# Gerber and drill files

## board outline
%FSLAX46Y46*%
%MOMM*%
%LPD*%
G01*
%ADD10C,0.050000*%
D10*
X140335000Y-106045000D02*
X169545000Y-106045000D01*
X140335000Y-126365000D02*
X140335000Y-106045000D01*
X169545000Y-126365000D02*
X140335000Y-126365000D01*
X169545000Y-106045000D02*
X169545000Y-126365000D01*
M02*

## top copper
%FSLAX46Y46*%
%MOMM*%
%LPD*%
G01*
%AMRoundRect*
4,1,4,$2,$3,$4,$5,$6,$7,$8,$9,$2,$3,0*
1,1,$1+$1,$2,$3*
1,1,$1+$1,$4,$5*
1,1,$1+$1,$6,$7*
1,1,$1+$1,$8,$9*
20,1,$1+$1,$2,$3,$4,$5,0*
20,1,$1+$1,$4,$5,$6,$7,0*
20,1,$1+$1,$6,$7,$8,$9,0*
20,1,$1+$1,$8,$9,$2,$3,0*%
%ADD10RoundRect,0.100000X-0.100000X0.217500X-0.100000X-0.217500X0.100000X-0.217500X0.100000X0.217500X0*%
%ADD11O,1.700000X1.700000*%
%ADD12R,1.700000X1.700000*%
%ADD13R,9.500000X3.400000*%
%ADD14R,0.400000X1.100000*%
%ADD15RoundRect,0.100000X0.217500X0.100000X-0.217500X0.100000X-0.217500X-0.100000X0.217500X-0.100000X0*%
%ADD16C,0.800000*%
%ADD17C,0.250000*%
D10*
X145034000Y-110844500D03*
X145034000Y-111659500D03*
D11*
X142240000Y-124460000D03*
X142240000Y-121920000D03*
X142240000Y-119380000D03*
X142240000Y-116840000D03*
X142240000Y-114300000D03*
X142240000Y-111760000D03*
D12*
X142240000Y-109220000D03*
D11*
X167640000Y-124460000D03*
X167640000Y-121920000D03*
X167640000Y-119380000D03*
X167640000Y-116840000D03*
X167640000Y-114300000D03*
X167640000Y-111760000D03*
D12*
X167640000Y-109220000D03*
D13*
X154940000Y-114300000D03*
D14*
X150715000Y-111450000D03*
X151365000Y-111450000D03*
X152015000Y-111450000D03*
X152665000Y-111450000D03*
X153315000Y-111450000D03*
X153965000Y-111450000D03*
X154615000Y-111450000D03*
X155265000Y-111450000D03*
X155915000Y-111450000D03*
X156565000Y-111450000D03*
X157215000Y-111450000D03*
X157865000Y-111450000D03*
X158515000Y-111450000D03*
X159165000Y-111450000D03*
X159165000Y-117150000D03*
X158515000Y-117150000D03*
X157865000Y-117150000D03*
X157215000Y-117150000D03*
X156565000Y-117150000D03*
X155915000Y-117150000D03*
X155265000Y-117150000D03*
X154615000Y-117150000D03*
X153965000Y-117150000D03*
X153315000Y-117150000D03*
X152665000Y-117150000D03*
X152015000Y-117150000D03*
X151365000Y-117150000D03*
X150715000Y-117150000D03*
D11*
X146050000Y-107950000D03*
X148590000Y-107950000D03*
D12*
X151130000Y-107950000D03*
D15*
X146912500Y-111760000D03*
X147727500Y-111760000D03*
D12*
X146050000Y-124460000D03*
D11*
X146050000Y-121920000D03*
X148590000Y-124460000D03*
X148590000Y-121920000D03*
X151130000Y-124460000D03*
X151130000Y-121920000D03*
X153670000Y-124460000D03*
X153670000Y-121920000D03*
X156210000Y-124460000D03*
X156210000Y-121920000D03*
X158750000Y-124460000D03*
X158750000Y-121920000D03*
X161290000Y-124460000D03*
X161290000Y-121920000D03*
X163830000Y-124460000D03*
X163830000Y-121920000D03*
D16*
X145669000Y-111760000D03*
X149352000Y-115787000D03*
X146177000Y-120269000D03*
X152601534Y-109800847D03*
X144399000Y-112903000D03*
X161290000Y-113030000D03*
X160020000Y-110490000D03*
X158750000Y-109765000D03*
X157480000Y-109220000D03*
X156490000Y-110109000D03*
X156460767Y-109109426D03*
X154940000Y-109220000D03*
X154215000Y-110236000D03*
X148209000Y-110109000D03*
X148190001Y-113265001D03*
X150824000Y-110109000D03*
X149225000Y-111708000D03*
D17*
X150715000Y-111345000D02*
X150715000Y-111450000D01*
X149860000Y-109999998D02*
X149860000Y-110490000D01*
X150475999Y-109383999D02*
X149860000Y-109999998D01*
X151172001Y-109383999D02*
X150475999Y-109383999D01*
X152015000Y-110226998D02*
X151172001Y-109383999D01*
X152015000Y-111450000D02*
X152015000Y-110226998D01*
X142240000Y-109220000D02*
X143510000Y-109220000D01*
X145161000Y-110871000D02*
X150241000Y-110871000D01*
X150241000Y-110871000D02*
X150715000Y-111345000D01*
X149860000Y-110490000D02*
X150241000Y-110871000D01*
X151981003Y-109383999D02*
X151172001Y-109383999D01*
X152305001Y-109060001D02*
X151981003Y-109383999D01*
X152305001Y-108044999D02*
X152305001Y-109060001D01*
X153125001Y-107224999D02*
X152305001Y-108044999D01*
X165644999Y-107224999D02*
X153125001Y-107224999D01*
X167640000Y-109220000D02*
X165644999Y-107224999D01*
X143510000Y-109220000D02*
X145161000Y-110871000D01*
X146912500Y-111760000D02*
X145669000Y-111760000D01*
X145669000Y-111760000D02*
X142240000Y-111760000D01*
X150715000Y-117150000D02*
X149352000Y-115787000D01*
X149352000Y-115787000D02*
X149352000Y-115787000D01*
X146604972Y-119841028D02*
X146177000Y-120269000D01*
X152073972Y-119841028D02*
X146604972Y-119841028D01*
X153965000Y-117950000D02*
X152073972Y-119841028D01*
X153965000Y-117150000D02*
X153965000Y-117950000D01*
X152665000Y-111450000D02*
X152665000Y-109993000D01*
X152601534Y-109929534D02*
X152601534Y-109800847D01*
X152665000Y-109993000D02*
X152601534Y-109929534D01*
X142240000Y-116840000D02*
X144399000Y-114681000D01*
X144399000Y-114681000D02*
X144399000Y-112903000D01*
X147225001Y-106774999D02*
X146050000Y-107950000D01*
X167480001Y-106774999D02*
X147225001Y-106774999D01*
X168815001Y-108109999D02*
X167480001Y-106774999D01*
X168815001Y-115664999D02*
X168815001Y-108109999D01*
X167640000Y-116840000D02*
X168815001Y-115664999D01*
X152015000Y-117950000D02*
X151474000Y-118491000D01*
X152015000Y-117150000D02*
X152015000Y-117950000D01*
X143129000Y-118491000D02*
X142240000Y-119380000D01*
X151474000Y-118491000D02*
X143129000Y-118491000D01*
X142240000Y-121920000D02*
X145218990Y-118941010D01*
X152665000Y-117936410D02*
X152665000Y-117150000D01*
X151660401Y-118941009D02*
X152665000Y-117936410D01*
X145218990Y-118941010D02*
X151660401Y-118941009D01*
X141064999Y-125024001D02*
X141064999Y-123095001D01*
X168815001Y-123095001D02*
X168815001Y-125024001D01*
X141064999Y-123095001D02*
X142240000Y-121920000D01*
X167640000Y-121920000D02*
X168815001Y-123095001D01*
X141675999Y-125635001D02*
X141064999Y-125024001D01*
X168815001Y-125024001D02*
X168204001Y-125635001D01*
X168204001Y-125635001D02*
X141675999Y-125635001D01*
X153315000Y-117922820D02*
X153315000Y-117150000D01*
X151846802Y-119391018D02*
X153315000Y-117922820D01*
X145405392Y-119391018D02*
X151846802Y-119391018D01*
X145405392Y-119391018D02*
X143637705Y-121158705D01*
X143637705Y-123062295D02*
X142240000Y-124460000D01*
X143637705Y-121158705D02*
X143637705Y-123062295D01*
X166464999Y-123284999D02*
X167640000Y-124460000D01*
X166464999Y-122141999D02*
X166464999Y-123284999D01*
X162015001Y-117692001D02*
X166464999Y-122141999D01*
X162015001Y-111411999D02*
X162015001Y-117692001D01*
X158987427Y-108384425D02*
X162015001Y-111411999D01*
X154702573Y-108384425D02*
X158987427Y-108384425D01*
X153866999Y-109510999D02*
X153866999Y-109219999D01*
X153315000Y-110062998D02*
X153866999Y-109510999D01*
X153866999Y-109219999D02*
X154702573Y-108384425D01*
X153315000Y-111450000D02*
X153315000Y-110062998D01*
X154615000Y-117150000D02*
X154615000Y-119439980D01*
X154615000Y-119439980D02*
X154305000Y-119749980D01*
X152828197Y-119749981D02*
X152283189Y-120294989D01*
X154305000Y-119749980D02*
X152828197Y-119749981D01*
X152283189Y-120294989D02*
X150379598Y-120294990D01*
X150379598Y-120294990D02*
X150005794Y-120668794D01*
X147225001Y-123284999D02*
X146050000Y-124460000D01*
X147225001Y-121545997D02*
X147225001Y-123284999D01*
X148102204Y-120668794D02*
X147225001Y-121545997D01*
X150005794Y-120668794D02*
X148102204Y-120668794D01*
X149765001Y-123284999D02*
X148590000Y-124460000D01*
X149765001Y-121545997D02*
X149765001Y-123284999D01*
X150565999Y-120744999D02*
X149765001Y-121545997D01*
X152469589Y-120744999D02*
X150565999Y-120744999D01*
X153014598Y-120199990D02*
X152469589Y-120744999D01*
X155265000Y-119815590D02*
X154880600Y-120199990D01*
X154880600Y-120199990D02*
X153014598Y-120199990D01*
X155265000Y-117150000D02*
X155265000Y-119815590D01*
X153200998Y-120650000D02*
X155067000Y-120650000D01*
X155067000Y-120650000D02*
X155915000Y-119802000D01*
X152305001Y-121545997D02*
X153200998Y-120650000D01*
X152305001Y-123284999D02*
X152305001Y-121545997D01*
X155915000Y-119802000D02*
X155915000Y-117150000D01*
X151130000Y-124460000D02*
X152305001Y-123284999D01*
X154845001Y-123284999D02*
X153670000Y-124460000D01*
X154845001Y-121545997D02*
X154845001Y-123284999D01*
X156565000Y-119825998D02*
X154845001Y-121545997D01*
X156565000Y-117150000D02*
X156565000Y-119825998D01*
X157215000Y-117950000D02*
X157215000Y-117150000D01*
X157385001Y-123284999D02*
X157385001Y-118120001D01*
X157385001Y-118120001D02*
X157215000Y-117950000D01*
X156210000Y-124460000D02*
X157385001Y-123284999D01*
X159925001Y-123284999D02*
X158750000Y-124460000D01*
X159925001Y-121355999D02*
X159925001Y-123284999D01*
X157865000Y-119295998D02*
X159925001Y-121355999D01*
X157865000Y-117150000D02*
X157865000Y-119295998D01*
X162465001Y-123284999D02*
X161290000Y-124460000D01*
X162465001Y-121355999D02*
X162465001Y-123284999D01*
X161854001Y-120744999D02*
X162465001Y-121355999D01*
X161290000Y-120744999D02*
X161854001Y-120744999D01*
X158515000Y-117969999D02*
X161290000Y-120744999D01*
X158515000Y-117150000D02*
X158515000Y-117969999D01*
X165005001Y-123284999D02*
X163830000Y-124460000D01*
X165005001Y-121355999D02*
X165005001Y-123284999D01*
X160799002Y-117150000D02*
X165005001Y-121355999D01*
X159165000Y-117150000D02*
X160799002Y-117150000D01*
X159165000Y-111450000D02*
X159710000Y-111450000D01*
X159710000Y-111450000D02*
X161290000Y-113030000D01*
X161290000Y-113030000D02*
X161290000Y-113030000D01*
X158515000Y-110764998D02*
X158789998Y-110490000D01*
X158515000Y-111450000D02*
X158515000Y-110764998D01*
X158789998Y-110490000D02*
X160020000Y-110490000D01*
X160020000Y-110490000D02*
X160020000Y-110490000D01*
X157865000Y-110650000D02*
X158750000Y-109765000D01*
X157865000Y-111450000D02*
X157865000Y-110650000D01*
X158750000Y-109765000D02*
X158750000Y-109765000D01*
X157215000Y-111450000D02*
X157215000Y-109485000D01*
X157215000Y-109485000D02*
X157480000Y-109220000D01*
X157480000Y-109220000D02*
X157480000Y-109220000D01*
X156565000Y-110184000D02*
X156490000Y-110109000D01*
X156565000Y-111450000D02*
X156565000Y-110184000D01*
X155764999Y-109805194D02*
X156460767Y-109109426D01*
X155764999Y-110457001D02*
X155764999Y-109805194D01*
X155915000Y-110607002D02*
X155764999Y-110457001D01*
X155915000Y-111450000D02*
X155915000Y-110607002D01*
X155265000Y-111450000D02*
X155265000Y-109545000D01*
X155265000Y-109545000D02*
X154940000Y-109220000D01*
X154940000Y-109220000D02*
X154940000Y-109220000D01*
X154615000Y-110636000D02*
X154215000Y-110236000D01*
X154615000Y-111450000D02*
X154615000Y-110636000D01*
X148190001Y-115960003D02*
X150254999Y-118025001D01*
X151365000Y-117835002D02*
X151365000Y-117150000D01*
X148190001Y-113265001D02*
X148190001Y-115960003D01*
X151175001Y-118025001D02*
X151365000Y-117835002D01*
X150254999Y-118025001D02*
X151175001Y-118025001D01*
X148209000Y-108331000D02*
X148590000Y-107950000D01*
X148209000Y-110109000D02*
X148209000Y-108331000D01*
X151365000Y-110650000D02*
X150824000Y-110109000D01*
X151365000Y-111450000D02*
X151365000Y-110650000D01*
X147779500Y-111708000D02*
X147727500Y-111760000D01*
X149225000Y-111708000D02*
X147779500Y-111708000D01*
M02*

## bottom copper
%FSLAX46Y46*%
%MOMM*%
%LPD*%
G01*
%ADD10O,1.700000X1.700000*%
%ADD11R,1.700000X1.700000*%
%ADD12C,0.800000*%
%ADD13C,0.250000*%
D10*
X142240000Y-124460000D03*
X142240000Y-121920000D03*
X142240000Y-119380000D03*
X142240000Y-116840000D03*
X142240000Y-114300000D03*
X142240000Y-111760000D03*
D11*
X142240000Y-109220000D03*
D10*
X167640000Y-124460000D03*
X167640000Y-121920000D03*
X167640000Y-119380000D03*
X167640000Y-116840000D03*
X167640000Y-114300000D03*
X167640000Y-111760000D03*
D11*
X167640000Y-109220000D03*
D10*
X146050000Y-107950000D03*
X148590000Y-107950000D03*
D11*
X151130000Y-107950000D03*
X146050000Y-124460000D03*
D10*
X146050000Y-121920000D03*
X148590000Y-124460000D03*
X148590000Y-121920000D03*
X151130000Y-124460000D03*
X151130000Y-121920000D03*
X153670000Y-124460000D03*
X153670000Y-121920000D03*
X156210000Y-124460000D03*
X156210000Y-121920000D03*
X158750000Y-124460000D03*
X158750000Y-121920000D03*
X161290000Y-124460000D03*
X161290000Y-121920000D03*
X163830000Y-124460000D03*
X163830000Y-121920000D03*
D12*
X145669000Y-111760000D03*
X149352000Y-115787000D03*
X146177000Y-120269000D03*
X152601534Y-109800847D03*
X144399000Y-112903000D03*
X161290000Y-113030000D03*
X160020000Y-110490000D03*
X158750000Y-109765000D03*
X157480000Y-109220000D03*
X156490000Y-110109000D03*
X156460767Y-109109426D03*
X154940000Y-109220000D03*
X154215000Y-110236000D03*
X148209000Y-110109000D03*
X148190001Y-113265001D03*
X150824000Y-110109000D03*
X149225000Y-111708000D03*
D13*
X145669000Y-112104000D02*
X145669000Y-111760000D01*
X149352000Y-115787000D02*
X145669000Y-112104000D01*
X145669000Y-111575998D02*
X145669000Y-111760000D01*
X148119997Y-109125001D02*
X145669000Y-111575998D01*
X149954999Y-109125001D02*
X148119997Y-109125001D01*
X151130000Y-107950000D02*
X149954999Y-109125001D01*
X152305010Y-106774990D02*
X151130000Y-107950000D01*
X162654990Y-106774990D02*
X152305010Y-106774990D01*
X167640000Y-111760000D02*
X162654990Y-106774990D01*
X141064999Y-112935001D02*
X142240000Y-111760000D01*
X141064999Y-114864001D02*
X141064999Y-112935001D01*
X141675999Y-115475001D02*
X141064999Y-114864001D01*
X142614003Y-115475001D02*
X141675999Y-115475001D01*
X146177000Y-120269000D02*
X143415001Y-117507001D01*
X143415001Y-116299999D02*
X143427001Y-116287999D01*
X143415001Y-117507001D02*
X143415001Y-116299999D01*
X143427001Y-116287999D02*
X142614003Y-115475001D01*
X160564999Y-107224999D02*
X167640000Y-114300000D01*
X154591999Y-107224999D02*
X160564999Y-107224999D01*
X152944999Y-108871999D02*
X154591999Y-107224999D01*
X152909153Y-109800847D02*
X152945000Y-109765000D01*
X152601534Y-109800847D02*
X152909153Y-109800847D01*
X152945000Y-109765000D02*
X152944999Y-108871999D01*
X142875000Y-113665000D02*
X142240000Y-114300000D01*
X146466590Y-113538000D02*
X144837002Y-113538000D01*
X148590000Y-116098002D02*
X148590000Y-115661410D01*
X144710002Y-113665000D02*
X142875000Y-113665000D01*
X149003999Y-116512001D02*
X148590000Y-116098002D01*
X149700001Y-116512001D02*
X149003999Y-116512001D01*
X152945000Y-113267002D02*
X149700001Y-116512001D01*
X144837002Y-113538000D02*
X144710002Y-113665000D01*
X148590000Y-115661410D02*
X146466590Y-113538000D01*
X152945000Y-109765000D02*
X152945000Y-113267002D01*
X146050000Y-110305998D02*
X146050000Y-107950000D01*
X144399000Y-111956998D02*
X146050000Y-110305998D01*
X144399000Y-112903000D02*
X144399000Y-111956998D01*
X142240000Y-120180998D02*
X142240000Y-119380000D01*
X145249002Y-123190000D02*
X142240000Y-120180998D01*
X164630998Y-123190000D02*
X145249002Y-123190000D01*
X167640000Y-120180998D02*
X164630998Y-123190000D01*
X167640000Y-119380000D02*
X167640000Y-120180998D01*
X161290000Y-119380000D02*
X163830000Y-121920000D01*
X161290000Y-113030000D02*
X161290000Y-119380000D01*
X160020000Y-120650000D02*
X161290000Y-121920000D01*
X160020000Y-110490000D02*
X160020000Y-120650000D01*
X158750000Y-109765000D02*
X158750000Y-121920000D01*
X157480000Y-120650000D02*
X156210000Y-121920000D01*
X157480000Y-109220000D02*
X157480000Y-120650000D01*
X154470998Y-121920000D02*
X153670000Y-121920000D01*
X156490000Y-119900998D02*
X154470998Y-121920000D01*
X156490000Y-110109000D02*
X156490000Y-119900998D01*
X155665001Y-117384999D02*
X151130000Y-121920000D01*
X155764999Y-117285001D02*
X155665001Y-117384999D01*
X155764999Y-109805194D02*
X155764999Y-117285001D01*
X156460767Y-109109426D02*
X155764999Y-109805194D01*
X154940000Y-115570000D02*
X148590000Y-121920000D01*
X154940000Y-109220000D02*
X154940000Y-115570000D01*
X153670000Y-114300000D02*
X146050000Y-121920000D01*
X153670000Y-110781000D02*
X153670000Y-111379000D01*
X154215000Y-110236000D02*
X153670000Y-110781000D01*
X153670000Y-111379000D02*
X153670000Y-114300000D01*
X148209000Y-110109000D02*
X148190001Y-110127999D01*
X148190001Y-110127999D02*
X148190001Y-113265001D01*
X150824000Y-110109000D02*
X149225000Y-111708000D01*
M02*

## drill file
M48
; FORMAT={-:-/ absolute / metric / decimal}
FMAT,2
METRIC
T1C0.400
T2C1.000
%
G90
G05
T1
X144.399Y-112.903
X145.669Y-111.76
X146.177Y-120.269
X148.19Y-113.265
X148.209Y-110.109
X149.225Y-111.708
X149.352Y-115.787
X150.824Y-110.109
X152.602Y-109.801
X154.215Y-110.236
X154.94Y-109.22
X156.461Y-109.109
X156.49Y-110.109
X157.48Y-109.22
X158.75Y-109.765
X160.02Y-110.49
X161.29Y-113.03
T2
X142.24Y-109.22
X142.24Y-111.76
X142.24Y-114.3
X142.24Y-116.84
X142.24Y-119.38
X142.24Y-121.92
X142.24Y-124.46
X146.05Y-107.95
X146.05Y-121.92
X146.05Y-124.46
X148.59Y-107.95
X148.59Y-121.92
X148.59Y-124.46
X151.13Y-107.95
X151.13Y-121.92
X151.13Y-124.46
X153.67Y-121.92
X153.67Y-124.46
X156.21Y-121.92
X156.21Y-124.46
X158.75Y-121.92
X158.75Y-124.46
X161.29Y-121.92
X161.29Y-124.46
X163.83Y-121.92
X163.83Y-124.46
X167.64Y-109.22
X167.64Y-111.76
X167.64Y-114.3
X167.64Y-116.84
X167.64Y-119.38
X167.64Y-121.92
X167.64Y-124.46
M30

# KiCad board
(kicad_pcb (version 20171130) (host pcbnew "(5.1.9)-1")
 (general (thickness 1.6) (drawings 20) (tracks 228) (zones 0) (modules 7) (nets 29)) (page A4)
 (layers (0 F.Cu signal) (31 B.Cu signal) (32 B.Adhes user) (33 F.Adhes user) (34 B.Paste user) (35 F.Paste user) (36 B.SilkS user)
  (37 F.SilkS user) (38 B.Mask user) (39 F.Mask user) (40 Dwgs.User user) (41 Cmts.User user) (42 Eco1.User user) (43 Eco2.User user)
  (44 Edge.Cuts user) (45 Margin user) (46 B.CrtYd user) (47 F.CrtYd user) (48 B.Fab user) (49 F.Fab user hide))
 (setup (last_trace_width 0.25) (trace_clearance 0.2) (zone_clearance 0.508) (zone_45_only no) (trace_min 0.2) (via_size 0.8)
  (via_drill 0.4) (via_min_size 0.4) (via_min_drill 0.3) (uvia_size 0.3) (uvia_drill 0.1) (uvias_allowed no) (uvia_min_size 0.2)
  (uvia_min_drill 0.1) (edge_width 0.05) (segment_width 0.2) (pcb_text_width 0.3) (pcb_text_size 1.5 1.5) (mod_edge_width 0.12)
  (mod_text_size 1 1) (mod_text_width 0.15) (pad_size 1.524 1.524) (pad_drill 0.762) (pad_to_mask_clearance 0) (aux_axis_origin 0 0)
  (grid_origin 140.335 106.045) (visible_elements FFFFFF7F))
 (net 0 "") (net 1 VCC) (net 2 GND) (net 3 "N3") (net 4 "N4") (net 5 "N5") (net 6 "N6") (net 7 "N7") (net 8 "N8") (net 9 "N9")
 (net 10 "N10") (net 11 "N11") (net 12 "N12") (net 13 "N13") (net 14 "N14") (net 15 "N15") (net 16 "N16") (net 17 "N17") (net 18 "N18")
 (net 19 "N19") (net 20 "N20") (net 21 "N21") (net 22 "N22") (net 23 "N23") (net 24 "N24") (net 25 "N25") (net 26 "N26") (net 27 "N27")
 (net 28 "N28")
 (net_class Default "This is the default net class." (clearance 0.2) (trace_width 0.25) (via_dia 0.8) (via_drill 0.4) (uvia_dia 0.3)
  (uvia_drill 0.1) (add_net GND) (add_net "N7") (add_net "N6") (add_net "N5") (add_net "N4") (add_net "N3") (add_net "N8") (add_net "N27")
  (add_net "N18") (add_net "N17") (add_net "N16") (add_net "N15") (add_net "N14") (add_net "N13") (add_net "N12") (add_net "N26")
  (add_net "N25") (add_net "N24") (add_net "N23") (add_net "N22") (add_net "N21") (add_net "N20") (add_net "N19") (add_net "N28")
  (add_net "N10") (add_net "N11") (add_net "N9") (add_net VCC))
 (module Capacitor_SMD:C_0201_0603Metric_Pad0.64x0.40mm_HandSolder (layer F.Cu) (at 145.034 111.252 270)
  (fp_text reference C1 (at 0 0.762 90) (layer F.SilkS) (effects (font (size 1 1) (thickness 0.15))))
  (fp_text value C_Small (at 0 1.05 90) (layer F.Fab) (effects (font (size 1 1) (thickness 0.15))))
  (pad "" smd roundrect (at -0.4325 0 270) (size 0.458 0.36) (layers F.Paste) (roundrect_rratio 0.25))
  (pad "" smd roundrect (at 0.4325 0 270) (size 0.458 0.36) (layers F.Paste) (roundrect_rratio 0.25))
  (pad 1 smd roundrect (at -0.4075 0 270) (size 0.635 0.4) (layers F.Cu F.Mask) (roundrect_rratio 0.25) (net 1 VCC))
  (pad 2 smd roundrect (at 0.4075 0 270) (size 0.635 0.4) (layers F.Cu F.Mask) (roundrect_rratio 0.25) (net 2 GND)))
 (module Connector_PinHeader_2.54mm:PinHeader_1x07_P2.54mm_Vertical (layer F.Cu) (at 142.24 109.22)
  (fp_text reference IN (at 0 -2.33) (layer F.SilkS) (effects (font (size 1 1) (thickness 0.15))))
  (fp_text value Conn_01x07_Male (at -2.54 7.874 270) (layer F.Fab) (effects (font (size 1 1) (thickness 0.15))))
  (pad 7 thru_hole oval (at 0 15.24) (size 1.7 1.7) (drill 1) (layers *.Cu *.Mask) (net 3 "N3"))
  (pad 6 thru_hole oval (at 0 12.7) (size 1.7 1.7) (drill 1) (layers *.Cu *.Mask) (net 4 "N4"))
  (pad 5 thru_hole oval (at 0 10.16) (size 1.7 1.7) (drill 1) (layers *.Cu *.Mask) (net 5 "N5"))
  (pad 4 thru_hole oval (at 0 7.62) (size 1.7 1.7) (drill 1) (layers *.Cu *.Mask) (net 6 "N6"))
  (pad 3 thru_hole oval (at 0 5.08) (size 1.7 1.7) (drill 1) (layers *.Cu *.Mask) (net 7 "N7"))
  (pad 2 thru_hole oval (at 0 2.54) (size 1.7 1.7) (drill 1) (layers *.Cu *.Mask) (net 2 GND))
  (pad 1 thru_hole rect (at 0 0) (size 1.7 1.7) (drill 1) (layers *.Cu *.Mask) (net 1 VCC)))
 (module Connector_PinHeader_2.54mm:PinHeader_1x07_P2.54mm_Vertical (layer F.Cu) (at 167.64 109.22)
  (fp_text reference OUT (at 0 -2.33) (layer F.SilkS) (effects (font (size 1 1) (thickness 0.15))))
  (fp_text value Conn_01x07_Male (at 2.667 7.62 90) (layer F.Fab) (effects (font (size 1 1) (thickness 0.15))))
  (pad 7 thru_hole oval (at 0 15.24) (size 1.7 1.7) (drill 1) (layers *.Cu *.Mask) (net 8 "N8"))
  (pad 6 thru_hole oval (at 0 12.7) (size 1.7 1.7) (drill 1) (layers *.Cu *.Mask) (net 4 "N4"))
  (pad 5 thru_hole oval (at 0 10.16) (size 1.7 1.7) (drill 1) (layers *.Cu *.Mask) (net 5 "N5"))
  (pad 4 thru_hole oval (at 0 7.62) (size 1.7 1.7) (drill 1) (layers *.Cu *.Mask) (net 6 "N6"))
  (pad 3 thru_hole oval (at 0 5.08) (size 1.7 1.7) (drill 1) (layers *.Cu *.Mask) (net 7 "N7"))
  (pad 2 thru_hole oval (at 0 2.54) (size 1.7 1.7) (drill 1) (layers *.Cu *.Mask) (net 2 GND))
  (pad 1 thru_hole rect (at 0 0) (size 1.7 1.7) (drill 1) (layers *.Cu *.Mask) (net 1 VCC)))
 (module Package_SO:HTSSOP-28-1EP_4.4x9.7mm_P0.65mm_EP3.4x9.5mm (layer F.Cu) (at 154.94 114.3 90)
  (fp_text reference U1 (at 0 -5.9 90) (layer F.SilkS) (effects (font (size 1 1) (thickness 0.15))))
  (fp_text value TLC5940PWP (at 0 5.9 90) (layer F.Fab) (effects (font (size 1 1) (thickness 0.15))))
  (pad "" smd rect (at -0.85 3.8 90) (size 1.4 1.6) (layers F.Paste))
  (pad "" smd rect (at 0.85 3.8 90) (size 1.4 1.6) (layers F.Paste))
  (pad "" smd rect (at -0.85 1.9 90) (size 1.4 1.6) (layers F.Paste))
  (pad "" smd rect (at 0.85 1.9 90) (size 1.4 1.6) (layers F.Paste))
  (pad "" smd rect (at -0.85 0 90) (size 1.4 1.6) (layers F.Paste))
  (pad "" smd rect (at 0.85 0 90) (size 1.4 1.6) (layers F.Paste))
  (pad "" smd rect (at -0.85 -1.9 90) (size 1.4 1.6) (layers F.Paste))
  (pad "" smd rect (at 0.85 -1.9 90) (size 1.4 1.6) (layers F.Paste))
  (pad "" smd rect (at 0.85 -3.8 90) (size 1.4 1.6) (layers F.Paste))
  (pad "" smd rect (at -0.85 -3.8 90) (size 1.4 1.6) (layers F.Paste))
  (pad 29 smd rect (at 0 0 90) (size 3.4 9.5) (layers F.Cu F.Mask) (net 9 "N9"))
  (pad 28 smd rect (at 2.85 -4.225 90) (size 1.1 0.4) (layers F.Cu F.Paste F.Mask) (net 1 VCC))
  (pad 27 smd rect (at 2.85 -3.575 90) (size 1.1 0.4) (layers F.Cu F.Paste F.Mask) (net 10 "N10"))
  (pad 26 smd rect (at 2.85 -2.925 90) (size 1.1 0.4) (layers F.Cu F.Paste F.Mask) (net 1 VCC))
  (pad 25 smd rect (at 2.85 -2.275 90) (size 1.1 0.4) (layers F.Cu F.Paste F.Mask) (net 7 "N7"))
  (pad 24 smd rect (at 2.85 -1.625 90) (size 1.1 0.4) (layers F.Cu F.Paste F.Mask) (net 8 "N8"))
  (pad 23 smd rect (at 2.85 -0.975 90) (size 1.1 0.4) (layers F.Cu F.Paste F.Mask) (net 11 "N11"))
  (pad 22 smd rect (at 2.85 -0.325 90) (size 1.1 0.4) (layers F.Cu F.Paste F.Mask) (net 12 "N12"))
  (pad 21 smd rect (at 2.85 0.325 90) (size 1.1 0.4) (layers F.Cu F.Paste F.Mask) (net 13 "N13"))
  (pad 20 smd rect (at 2.85 0.975 90) (size 1.1 0.4) (layers F.Cu F.Paste F.Mask) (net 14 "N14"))
  (pad 19 smd rect (at 2.85 1.625 90) (size 1.1 0.4) (layers F.Cu F.Paste F.Mask) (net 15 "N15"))
  (pad 18 smd rect (at 2.85 2.275 90) (size 1.1 0.4) (layers F.Cu F.Paste F.Mask) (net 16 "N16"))
  (pad 17 smd rect (at 2.85 2.925 90) (size 1.1 0.4) (layers F.Cu F.Paste F.Mask) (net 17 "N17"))
  (pad 16 smd rect (at 2.85 3.575 90) (size 1.1 0.4) (layers F.Cu F.Paste F.Mask) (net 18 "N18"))
  (pad 15 smd rect (at 2.85 4.225 90) (size 1.1 0.4) (layers F.Cu F.Paste F.Mask) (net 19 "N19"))
  (pad 14 smd rect (at -2.85 4.225 90) (size 1.1 0.4) (layers F.Cu F.Paste F.Mask) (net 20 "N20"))
  (pad 13 smd rect (at -2.85 3.575 90) (size 1.1 0.4) (layers F.Cu F.Paste F.Mask) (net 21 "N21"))
  (pad 12 smd rect (at -2.85 2.925 90) (size 1.1 0.4) (layers F.Cu F.Paste F.Mask) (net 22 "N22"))
  (pad 11 smd rect (at -2.85 2.275 90) (size 1.1 0.4) (layers F.Cu F.Paste F.Mask) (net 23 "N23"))
  (pad 10 smd rect (at -2.85 1.625 90) (size 1.1 0.4) (layers F.Cu F.Paste F.Mask) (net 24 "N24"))
  (pad 9 smd rect (at -2.85 0.975 90) (size 1.1 0.4) (layers F.Cu F.Paste F.Mask) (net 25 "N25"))
  (pad 8 smd rect (at -2.85 0.325 90) (size 1.1 0.4) (layers F.Cu F.Paste F.Mask) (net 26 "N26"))
  (pad 7 smd rect (at -2.85 -0.325 90) (size 1.1 0.4) (layers F.Cu F.Paste F.Mask) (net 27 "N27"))
  (pad 6 smd rect (at -2.85 -0.975 90) (size 1.1 0.4) (layers F.Cu F.Paste F.Mask) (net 2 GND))
  (pad 5 smd rect (at -2.85 -1.625 90) (size 1.1 0.4) (layers F.Cu F.Paste F.Mask) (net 3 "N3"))
  (pad 4 smd rect (at -2.85 -2.275 90) (size 1.1 0.4) (layers F.Cu F.Paste F.Mask) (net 4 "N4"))
  (pad 3 smd rect (at -2.85 -2.925 90) (size 1.1 0.4) (layers F.Cu F.Paste F.Mask) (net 5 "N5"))
  (pad 2 smd rect (at -2.85 -3.575 90) (size 1.1 0.4) (layers F.Cu F.Paste F.Mask) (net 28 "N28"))
  (pad 1 smd rect (at -2.85 -4.225 90) (size 1.1 0.4) (layers F.Cu F.Paste F.Mask) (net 2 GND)))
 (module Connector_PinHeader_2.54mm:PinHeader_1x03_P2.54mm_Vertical (layer F.Cu) (at 151.13 107.95 270)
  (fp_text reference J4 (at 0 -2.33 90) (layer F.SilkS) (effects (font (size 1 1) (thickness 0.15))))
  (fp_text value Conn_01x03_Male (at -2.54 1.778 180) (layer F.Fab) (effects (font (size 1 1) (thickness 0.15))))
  (pad 3 thru_hole oval (at 0 5.08 270) (size 1.7 1.7) (drill 1) (layers *.Cu *.Mask) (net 6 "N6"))
  (pad 2 thru_hole oval (at 0 2.54 270) (size 1.7 1.7) (drill 1) (layers *.Cu *.Mask) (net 28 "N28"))
  (pad 1 thru_hole rect (at 0 0 270) (size 1.7 1.7) (drill 1) (layers *.Cu *.Mask) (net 2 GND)))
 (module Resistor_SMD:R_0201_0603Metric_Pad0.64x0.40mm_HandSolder (layer F.Cu) (at 147.32 111.76 180)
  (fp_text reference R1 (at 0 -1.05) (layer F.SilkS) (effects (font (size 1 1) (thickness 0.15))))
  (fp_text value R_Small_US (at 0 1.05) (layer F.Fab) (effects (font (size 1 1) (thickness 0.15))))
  (pad 2 smd roundrect (at 0.4075 0 180) (size 0.635 0.4) (layers F.Cu F.Mask) (roundrect_rratio 0.25) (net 2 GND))
  (pad 1 smd roundrect (at -0.4075 0 180) (size 0.635 0.4) (layers F.Cu F.Mask) (roundrect_rratio 0.25) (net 10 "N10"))
  (pad "" smd roundrect (at 0.4325 0 180) (size 0.458 0.36) (layers F.Paste) (roundrect_rratio 0.25))
  (pad "" smd roundrect (at -0.4325 0 180) (size 0.458 0.36) (layers F.Paste) (roundrect_rratio 0.25)))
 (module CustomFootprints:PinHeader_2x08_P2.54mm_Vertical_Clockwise (layer F.Cu) (at 146.05 124.46 90)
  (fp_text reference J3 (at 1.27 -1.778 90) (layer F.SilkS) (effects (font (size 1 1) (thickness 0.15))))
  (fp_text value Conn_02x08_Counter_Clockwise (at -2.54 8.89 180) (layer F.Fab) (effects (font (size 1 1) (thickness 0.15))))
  (pad 1 thru_hole rect (at 0 0 90) (size 1.7 1.7) (drill 1) (layers *.Cu *.Mask) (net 27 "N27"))
  (pad 16 thru_hole oval (at 2.54 0 90) (size 1.7 1.7) (drill 1) (layers *.Cu *.Mask) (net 12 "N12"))
  (pad 2 thru_hole oval (at 0 2.54 90) (size 1.7 1.7) (drill 1) (layers *.Cu *.Mask) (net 26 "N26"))
  (pad 15 thru_hole oval (at 2.54 2.54 90) (size 1.7 1.7) (drill 1) (layers *.Cu *.Mask) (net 13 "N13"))
  (pad 3 thru_hole oval (at 0 5.08 90) (size 1.7 1.7) (drill 1) (layers *.Cu *.Mask) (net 25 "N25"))
  (pad 14 thru_hole oval (at 2.54 5.08 90) (size 1.7 1.7) (drill 1) (layers *.Cu *.Mask) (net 14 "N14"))
  (pad 4 thru_hole oval (at 0 7.62 90) (size 1.7 1.7) (drill 1) (layers *.Cu *.Mask) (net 24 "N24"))
  (pad 13 thru_hole oval (at 2.54 7.62 90) (size 1.7 1.7) (drill 1) (layers *.Cu *.Mask) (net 15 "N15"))
  (pad 5 thru_hole oval (at 0 10.16 90) (size 1.7 1.7) (drill 1) (layers *.Cu *.Mask) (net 23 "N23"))
  (pad 12 thru_hole oval (at 2.54 10.16 90) (size 1.7 1.7) (drill 1) (layers *.Cu *.Mask) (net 16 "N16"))
  (pad 6 thru_hole oval (at 0 12.7 90) (size 1.7 1.7) (drill 1) (layers *.Cu *.Mask) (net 22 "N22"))
  (pad 11 thru_hole oval (at 2.54 12.7 90) (size 1.7 1.7) (drill 1) (layers *.Cu *.Mask) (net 17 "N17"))
  (pad 7 thru_hole oval (at 0 15.24 90) (size 1.7 1.7) (drill 1) (layers *.Cu *.Mask) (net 21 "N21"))
  (pad 10 thru_hole oval (at 2.54 15.24 90) (size 1.7 1.7) (drill 1) (layers *.Cu *.Mask) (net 18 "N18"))
  (pad 8 thru_hole oval (at 0 17.78 90) (size 1.7 1.7) (drill 1) (layers *.Cu *.Mask) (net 20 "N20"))
  (pad 9 thru_hole oval (at 2.54 17.78 90) (size 1.7 1.7) (drill 1) (layers *.Cu *.Mask) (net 19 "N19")))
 (gr_line (start 140.335 106.045) (end 169.545 106.045) (layer Edge.Cuts) (width 0.05))
 (gr_line (start 140.335 126.365) (end 140.335 106.045) (layer Edge.Cuts) (width 0.05))
 (gr_line (start 169.545 126.365) (end 140.335 126.365) (layer Edge.Cuts) (width 0.05))
 (gr_line (start 169.545 106.045) (end 169.545 126.365) (layer Edge.Cuts) (width 0.05))
 (segment (start 150.715 111.345) (end 150.715 111.45) (width 0.25) (layer F.Cu) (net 1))
 (segment (start 149.86 109.999998) (end 149.86 110.49) (width 0.25) (layer F.Cu) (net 1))
 (segment (start 150.475999 109.383999) (end 149.86 109.999998) (width 0.25) (layer F.Cu) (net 1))
 (segment (start 151.172001 109.383999) (end 150.475999 109.383999) (width 0.25) (layer F.Cu) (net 1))
 (segment (start 152.015 110.226998) (end 151.172001 109.383999) (width 0.25) (layer F.Cu) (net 1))
 (segment (start 152.015 111.45) (end 152.015 110.226998) (width 0.25) (layer F.Cu) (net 1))
 (segment (start 142.24 109.22) (end 143.51 109.22) (width 0.25) (layer F.Cu) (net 1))
 (segment (start 145.161 110.871) (end 150.241 110.871) (width 0.25) (layer F.Cu) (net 1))
 (segment (start 150.241 110.871) (end 150.715 111.345) (width 0.25) (layer F.Cu) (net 1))
 (segment (start 149.86 110.49) (end 150.241 110.871) (width 0.25) (layer F.Cu) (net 1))
 (segment (start 151.981003 109.383999) (end 151.172001 109.383999) (width 0.25) (layer F.Cu) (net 1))
 (segment (start 152.305001 109.060001) (end 151.981003 109.383999) (width 0.25) (layer F.Cu) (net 1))
 (segment (start 152.305001 108.044999) (end 152.305001 109.060001) (width 0.25) (layer F.Cu) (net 1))
 (segment (start 153.125001 107.224999) (end 152.305001 108.044999) (width 0.25) (layer F.Cu) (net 1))
 (segment (start 165.644999 107.224999) (end 153.125001 107.224999) (width 0.25) (layer F.Cu) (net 1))
 (segment (start 167.64 109.22) (end 165.644999 107.224999) (width 0.25) (layer F.Cu) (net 1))
 (segment (start 143.51 109.22) (end 145.161 110.871) (width 0.25) (layer F.Cu) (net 1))
 (segment (start 146.9125 111.76) (end 145.669 111.76) (width 0.25) (layer F.Cu) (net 2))
 (segment (start 145.669 111.76) (end 142.24 111.76) (width 0.25) (layer F.Cu) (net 2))
 (via (at 145.669 111.76) (size 0.8) (drill 0.4) (layers F.Cu B.Cu) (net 2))
 (segment (start 150.715 117.15) (end 149.352 115.787) (width 0.25) (layer F.Cu) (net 2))
 (segment (start 149.352 115.787) (end 149.352 115.787) (width 0.25) (layer F.Cu) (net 2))
 (via (at 149.352 115.787) (size 0.8) (drill 0.4) (layers F.Cu B.Cu) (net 2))
 (segment (start 145.669 112.104) (end 145.669 111.76) (width 0.25) (layer B.Cu) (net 2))
 (segment (start 149.352 115.787) (end 145.669 112.104) (width 0.25) (layer B.Cu) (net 2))
 (segment (start 145.669 111.575998) (end 145.669 111.76) (width 0.25) (layer B.Cu) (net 2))
 (segment (start 148.119997 109.125001) (end 145.669 111.575998) (width 0.25) (layer B.Cu) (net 2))
 (segment (start 149.954999 109.125001) (end 148.119997 109.125001) (width 0.25) (layer B.Cu) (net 2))
 (segment (start 151.13 107.95) (end 149.954999 109.125001) (width 0.25) (layer B.Cu) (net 2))
 (segment (start 152.30501 106.77499) (end 151.13 107.95) (width 0.25) (layer B.Cu) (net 2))
 (segment (start 162.65499 106.77499) (end 152.30501 106.77499) (width 0.25) (layer B.Cu) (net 2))
 (segment (start 167.64 111.76) (end 162.65499 106.77499) (width 0.25) (layer B.Cu) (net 2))
 (segment (start 146.604972 119.841028) (end 146.177 120.269) (width 0.25) (layer F.Cu) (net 2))
 (segment (start 152.073972 119.841028) (end 146.604972 119.841028) (width 0.25) (layer F.Cu) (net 2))
 (segment (start 153.965 117.95) (end 152.073972 119.841028) (width 0.25) (layer F.Cu) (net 2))
 (via (at 146.177 120.269) (size 0.8) (drill 0.4) (layers F.Cu B.Cu) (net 2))
 (segment (start 153.965 117.15) (end 153.965 117.95) (width 0.25) (layer F.Cu) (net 2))
 (segment (start 141.064999 112.935001) (end 142.24 111.76) (width 0.25) (layer B.Cu) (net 2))
 (segment (start 141.064999 114.864001) (end 141.064999 112.935001) (width 0.25) (layer B.Cu) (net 2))
 (segment (start 141.675999 115.475001) (end 141.064999 114.864001) (width 0.25) (layer B.Cu) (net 2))
 (segment (start 142.614003 115.475001) (end 141.675999 115.475001) (width 0.25) (layer B.Cu) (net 2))
 (segment (start 146.177 120.269) (end 143.415001 117.507001) (width 0.25) (layer B.Cu) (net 2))
 (segment (start 143.415001 116.299999) (end 143.427001 116.287999) (width 0.25) (layer B.Cu) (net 2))
 (segment (start 143.415001 117.507001) (end 143.415001 116.299999) (width 0.25) (layer B.Cu) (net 2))
 (segment (start 143.427001 116.287999) (end 142.614003 115.475001) (width 0.25) (layer B.Cu) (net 2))
 (segment (start 160.564999 107.224999) (end 167.64 114.3) (width 0.25) (layer B.Cu) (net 7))
 (segment (start 154.591999 107.224999) (end 160.564999 107.224999) (width 0.25) (layer B.Cu) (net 7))
 (segment (start 152.944999 108.871999) (end 154.591999 107.224999) (width 0.25) (layer B.Cu) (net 7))
 (segment (start 152.665 111.45) (end 152.665 109.993) (width 0.25) (layer F.Cu) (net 7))
 (via (at 152.601534 109.800847) (size 0.8) (drill 0.4) (layers F.Cu B.Cu) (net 7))
 (segment (start 152.601534 109.929534) (end 152.601534 109.800847) (width 0.25) (layer F.Cu) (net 7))
 (segment (start 152.665 109.993) (end 152.601534 109.929534) (width 0.25) (layer F.Cu) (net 7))
 (segment (start 152.909153 109.800847) (end 152.945 109.765) (width 0.25) (layer B.Cu) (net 7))
 (segment (start 152.601534 109.800847) (end 152.909153 109.800847) (width 0.25) (layer B.Cu) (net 7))
 (segment (start 152.945 109.765) (end 152.944999 108.871999) (width 0.25) (layer B.Cu) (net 7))
 (segment (start 142.875 113.665) (end 142.24 114.3) (width 0.25) (layer B.Cu) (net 7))
 (segment (start 146.46659 113.538) (end 144.837002 113.538) (width 0.25) (layer B.Cu) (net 7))
 (segment (start 148.59 116.098002) (end 148.59 115.66141) (width 0.25) (layer B.Cu) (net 7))
 (segment (start 144.710002 113.665) (end 142.875 113.665) (width 0.25) (layer B.Cu) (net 7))
 (segment (start 149.003999 116.512001) (end 148.59 116.098002) (width 0.25) (layer B.Cu) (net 7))
 (segment (start 149.700001 116.512001) (end 149.003999 116.512001) (width 0.25) (layer B.Cu) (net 7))
 (segment (start 152.945 113.267002) (end 149.700001 116.512001) (width 0.25) (layer B.Cu) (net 7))
 (segment (start 144.837002 113.538) (end 144.710002 113.665) (width 0.25) (layer B.Cu) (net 7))
 (segment (start 148.59 115.66141) (end 146.46659 113.538) (width 0.25) (layer B.Cu) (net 7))
 (segment (start 152.945 109.765) (end 152.945 113.267002) (width 0.25) (layer B.Cu) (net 7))
 (segment (start 142.24 116.84) (end 144.399 114.681) (width 0.25) (layer F.Cu) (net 6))
 (segment (start 144.399 114.681) (end 144.399 112.903) (width 0.25) (layer F.Cu) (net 6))
 (via (at 144.399 112.903) (size 0.8) (drill 0.4) (layers F.Cu B.Cu) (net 6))
 (segment (start 146.05 110.305998) (end 146.05 107.95) (width 0.25) (layer B.Cu) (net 6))
 (segment (start 144.399 111.956998) (end 146.05 110.305998) (width 0.25) (layer B.Cu) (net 6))
 (segment (start 144.399 112.903) (end 144.399 111.956998) (width 0.25) (layer B.Cu) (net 6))
 (segment (start 147.225001 106.774999) (end 146.05 107.95) (width 0.25) (layer F.Cu) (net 6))
 (segment (start 167.480001 106.774999) (end 147.225001 106.774999) (width 0.25) (layer F.Cu) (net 6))
 (segment (start 168.815001 108.109999) (end 167.480001 106.774999) (width 0.25) (layer F.Cu) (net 6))
 (segment (start 168.815001 115.664999) (end 168.815001 108.109999) (width 0.25) (layer F.Cu) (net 6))
 (segment (start 167.64 116.84) (end 168.815001 115.664999) (width 0.25) (layer F.Cu) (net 6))
 (segment (start 152.015 117.95) (end 151.474 118.491) (width 0.25) (layer F.Cu) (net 5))
 (segment (start 152.015 117.15) (end 152.015 117.95) (width 0.25) (layer F.Cu) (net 5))
 (segment (start 143.129 118.491) (end 142.24 119.38) (width 0.25) (layer F.Cu) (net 5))
 (segment (start 151.474 118.491) (end 143.129 118.491) (width 0.25) (layer F.Cu) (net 5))
 (segment (start 142.24 120.180998) (end 142.24 119.38) (width 0.25) (layer B.Cu) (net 5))
 (segment (start 145.249002 123.19) (end 142.24 120.180998) (width 0.25) (layer B.Cu) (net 5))
 (segment (start 164.630998 123.19) (end 145.249002 123.19) (width 0.25) (layer B.Cu) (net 5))
 (segment (start 167.64 120.180998) (end 164.630998 123.19) (width 0.25) (layer B.Cu) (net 5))
 (segment (start 167.64 119.38) (end 167.64 120.180998) (width 0.25) (layer B.Cu) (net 5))
 (segment (start 142.24 121.92) (end 145.21899 118.94101) (width 0.25) (layer F.Cu) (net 4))
 (segment (start 152.665 117.93641) (end 152.665 117.15) (width 0.25) (layer F.Cu) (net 4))
 (segment (start 151.660401 118.941009) (end 152.665 117.93641) (width 0.25) (layer F.Cu) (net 4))
 (segment (start 145.21899 118.94101) (end 151.660401 118.941009) (width 0.25) (layer F.Cu) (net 4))
 (segment (start 141.064999 125.024001) (end 141.064999 123.095001) (width 0.25) (layer F.Cu) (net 4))
 (segment (start 168.815001 123.095001) (end 168.815001 125.024001) (width 0.25) (layer F.Cu) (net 4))
 (segment (start 141.064999 123.095001) (end 142.24 121.92) (width 0.25) (layer F.Cu) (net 4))
 (segment (start 167.64 121.92) (end 168.815001 123.095001) (width 0.25) (layer F.Cu) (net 4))
 (segment (start 141.675999 125.635001) (end 141.064999 125.024001) (width 0.25) (layer F.Cu) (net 4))
 (segment (start 168.815001 125.024001) (end 168.204001 125.635001) (width 0.25) (layer F.Cu) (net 4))
 (segment (start 168.204001 125.635001) (end 141.675999 125.635001) (width 0.25) (layer F.Cu) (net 4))
 (segment (start 153.315 117.92282) (end 153.315 117.15) (width 0.25) (layer F.Cu) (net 3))
 (segment (start 151.846802 119.391018) (end 153.315 117.92282) (width 0.25) (layer F.Cu) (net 3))
 (segment (start 145.405392 119.391018) (end 151.846802 119.391018) (width 0.25) (layer F.Cu) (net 3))
 (segment (start 145.405392 119.391018) (end 143.637705 121.158705) (width 0.25) (layer F.Cu) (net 3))
 (segment (start 143.637705 123.062295) (end 142.24 124.46) (width 0.25) (layer F.Cu) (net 3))
 (segment (start 143.637705 121.158705) (end 143.637705 123.062295) (width 0.25) (layer F.Cu) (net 3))
 (segment (start 166.464999 123.284999) (end 167.64 124.46) (width 0.25) (layer F.Cu) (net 8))
 (segment (start 166.464999 122.141999) (end 166.464999 123.284999) (width 0.25) (layer F.Cu) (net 8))
 (segment (start 162.015001 117.692001) (end 166.464999 122.141999) (width 0.25) (layer F.Cu) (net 8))
 (segment (start 162.015001 111.411999) (end 162.015001 117.692001) (width 0.25) (layer F.Cu) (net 8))
 (segment (start 158.987427 108.384425) (end 162.015001 111.411999) (width 0.25) (layer F.Cu) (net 8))
 (segment (start 154.702573 108.384425) (end 158.987427 108.384425) (width 0.25) (layer F.Cu) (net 8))
 (segment (start 153.866999 109.510999) (end 153.866999 109.219999) (width 0.25) (layer F.Cu) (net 8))
 (segment (start 153.315 110.062998) (end 153.866999 109.510999) (width 0.25) (layer F.Cu) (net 8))
 (segment (start 153.866999 109.219999) (end 154.702573 108.384425) (width 0.25) (layer F.Cu) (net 8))
 (segment (start 153.315 111.45) (end 153.315 110.062998) (width 0.25) (layer F.Cu) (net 8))
 (segment (start 154.615 117.15) (end 154.615 119.43998) (width 0.25) (layer F.Cu) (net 27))
 (segment (start 154.615 119.43998) (end 154.305 119.74998) (width 0.25) (layer F.Cu) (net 27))
 (segment (start 152.828197 119.749981) (end 152.283189 120.294989) (width 0.25) (layer F.Cu) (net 27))
 (segment (start 154.305 119.74998) (end 152.828197 119.749981) (width 0.25) (layer F.Cu) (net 27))
 (segment (start 152.283189 120.294989) (end 150.379598 120.29499) (width 0.25) (layer F.Cu) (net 27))
 (segment (start 150.379598 120.29499) (end 150.005794 120.668794) (width 0.25) (layer F.Cu) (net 27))
 (segment (start 147.225001 123.284999) (end 146.05 124.46) (width 0.25) (layer F.Cu) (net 27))
 (segment (start 147.225001 121.545997) (end 147.225001 123.284999) (width 0.25) (layer F.Cu) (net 27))
 (segment (start 148.102204 120.668794) (end 147.225001 121.545997) (width 0.25) (layer F.Cu) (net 27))
 (segment (start 150.005794 120.668794) (end 148.102204 120.668794) (width 0.25) (layer F.Cu) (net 27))
 (segment (start 149.765001 123.284999) (end 148.59 124.46) (width 0.25) (layer F.Cu) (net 26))
 (segment (start 149.765001 121.545997) (end 149.765001 123.284999) (width 0.25) (layer F.Cu) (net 26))
 (segment (start 150.565999 120.744999) (end 149.765001 121.545997) (width 0.25) (layer F.Cu) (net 26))
 (segment (start 152.469589 120.744999) (end 150.565999 120.744999) (width 0.25) (layer F.Cu) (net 26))
 (segment (start 153.014598 120.19999) (end 152.469589 120.744999) (width 0.25) (layer F.Cu) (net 26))
 (segment (start 155.265 119.81559) (end 154.8806 120.19999) (width 0.25) (layer F.Cu) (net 26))
 (segment (start 154.8806 120.19999) (end 153.014598 120.19999) (width 0.25) (layer F.Cu) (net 26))
 (segment (start 155.265 117.15) (end 155.265 119.81559) (width 0.25) (layer F.Cu) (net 26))
 (segment (start 153.200998 120.65) (end 155.067 120.65) (width 0.25) (layer F.Cu) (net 25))
 (segment (start 155.067 120.65) (end 155.915 119.802) (width 0.25) (layer F.Cu) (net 25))
 (segment (start 152.305001 121.545997) (end 153.200998 120.65) (width 0.25) (layer F.Cu) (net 25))
 (segment (start 152.305001 123.284999) (end 152.305001 121.545997) (width 0.25) (layer F.Cu) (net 25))
 (segment (start 155.915 119.802) (end 155.915 117.15) (width 0.25) (layer F.Cu) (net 25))
 (segment (start 151.13 124.46) (end 152.305001 123.284999) (width 0.25) (layer F.Cu) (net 25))
 (segment (start 154.845001 123.284999) (end 153.67 124.46) (width 0.25) (layer F.Cu) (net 24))
 (segment (start 154.845001 121.545997) (end 154.845001 123.284999) (width 0.25) (layer F.Cu) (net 24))
 (segment (start 156.565 119.825998) (end 154.845001 121.545997) (width 0.25) (layer F.Cu) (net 24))
 (segment (start 156.565 117.15) (end 156.565 119.825998) (width 0.25) (layer F.Cu) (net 24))
 (segment (start 157.215 117.95) (end 157.215 117.15) (width 0.25) (layer F.Cu) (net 23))
 (segment (start 157.385001 123.284999) (end 157.385001 118.120001) (width 0.25) (layer F.Cu) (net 23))
 (segment (start 157.385001 118.120001) (end 157.215 117.95) (width 0.25) (layer F.Cu) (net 23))
 (segment (start 156.21 124.46) (end 157.385001 123.284999) (width 0.25) (layer F.Cu) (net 23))
 (segment (start 159.925001 123.284999) (end 158.75 124.46) (width 0.25) (layer F.Cu) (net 22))
 (segment (start 159.925001 121.355999) (end 159.925001 123.284999) (width 0.25) (layer F.Cu) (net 22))
 (segment (start 157.865 119.295998) (end 159.925001 121.355999) (width 0.25) (layer F.Cu) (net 22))
 (segment (start 157.865 117.15) (end 157.865 119.295998) (width 0.25) (layer F.Cu) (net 22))
 (segment (start 162.465001 123.284999) (end 161.29 124.46) (width 0.25) (layer F.Cu) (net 21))
 (segment (start 162.465001 121.355999) (end 162.465001 123.284999) (width 0.25) (layer F.Cu) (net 21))
 (segment (start 161.854001 120.744999) (end 162.465001 121.355999) (width 0.25) (layer F.Cu) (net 21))
 (segment (start 161.29 120.744999) (end 161.854001 120.744999) (width 0.25) (layer F.Cu) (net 21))
 (segment (start 158.515 117.969999) (end 161.29 120.744999) (width 0.25) (layer F.Cu) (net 21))
 (segment (start 158.515 117.15) (end 158.515 117.969999) (width 0.25) (layer F.Cu) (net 21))
 (segment (start 165.005001 123.284999) (end 163.83 124.46) (width 0.25) (layer F.Cu) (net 20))
 (segment (start 165.005001 121.355999) (end 165.005001 123.284999) (width 0.25) (layer F.Cu) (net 20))
 (segment (start 160.799002 117.15) (end 165.005001 121.355999) (width 0.25) (layer F.Cu) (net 20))
 (segment (start 159.165 117.15) (end 160.799002 117.15) (width 0.25) (layer F.Cu) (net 20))
 (segment (start 159.165 111.45) (end 159.71 111.45) (width 0.25) (layer F.Cu) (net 19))
 (segment (start 159.71 111.45) (end 161.29 113.03) (width 0.25) (layer F.Cu) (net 19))
 (segment (start 161.29 113.03) (end 161.29 113.03) (width 0.25) (layer F.Cu) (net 19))
 (via (at 161.29 113.03) (size 0.8) (drill 0.4) (layers F.Cu B.Cu) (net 19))
 (segment (start 161.29 119.38) (end 163.83 121.92) (width 0.25) (layer B.Cu) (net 19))
 (segment (start 161.29 113.03) (end 161.29 119.38) (width 0.25) (layer B.Cu) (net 19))
 (segment (start 158.515 110.764998) (end 158.789998 110.49) (width 0.25) (layer F.Cu) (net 18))
 (segment (start 158.515 111.45) (end 158.515 110.764998) (width 0.25) (layer F.Cu) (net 18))
 (segment (start 158.789998 110.49) (end 160.02 110.49) (width 0.25) (layer F.Cu) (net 18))
 (segment (start 160.02 110.49) (end 160.02 110.49) (width 0.25) (layer F.Cu) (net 18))
 (via (at 160.02 110.49) (size 0.8) (drill 0.4) (layers F.Cu B.Cu) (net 18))
 (segment (start 160.02 120.65) (end 161.29 121.92) (width 0.25) (layer B.Cu) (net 18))
 (segment (start 160.02 110.49) (end 160.02 120.65) (width 0.25) (layer B.Cu) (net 18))
 (segment (start 157.865 110.65) (end 158.75 109.765) (width 0.25) (layer F.Cu) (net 17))
 (segment (start 157.865 111.45) (end 157.865 110.65) (width 0.25) (layer F.Cu) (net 17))
 (segment (start 158.75 109.765) (end 158.75 109.765) (width 0.25) (layer F.Cu) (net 17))
 (via (at 158.75 109.765) (size 0.8) (drill 0.4) (layers F.Cu B.Cu) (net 17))
 (segment (start 158.75 109.765) (end 158.75 121.92) (width 0.25) (layer B.Cu) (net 17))
 (segment (start 157.215 111.45) (end 157.215 109.485) (width 0.25) (layer F.Cu) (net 16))
 (segment (start 157.215 109.485) (end 157.48 109.22) (width 0.25) (layer F.Cu) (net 16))
 (segment (start 157.48 109.22) (end 157.48 109.22) (width 0.25) (layer F.Cu) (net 16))
 (via (at 157.48 109.22) (size 0.8) (drill 0.4) (layers F.Cu B.Cu) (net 16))
 (segment (start 157.48 120.65) (end 156.21 121.92) (width 0.25) (layer B.Cu) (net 16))
 (segment (start 157.48 109.22) (end 157.48 120.65) (width 0.25) (layer B.Cu) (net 16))
 (via (at 156.49 110.109) (size 0.8) (drill 0.4) (layers F.Cu B.Cu) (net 15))
 (segment (start 156.565 110.184) (end 156.49 110.109) (width 0.25) (layer F.Cu) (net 15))
 (segment (start 156.565 111.45) (end 156.565 110.184) (width 0.25) (layer F.Cu) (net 15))
 (segment (start 154.470998 121.92) (end 153.67 121.92) (width 0.25) (layer B.Cu) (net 15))
 (segment (start 156.49 119.900998) (end 154.470998 121.92) (width 0.25) (layer B.Cu) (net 15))
 (segment (start 156.49 110.109) (end 156.49 119.900998) (width 0.25) (layer B.Cu) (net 15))
 (segment (start 155.665001 117.384999) (end 151.13 121.92) (width 0.25) (layer B.Cu) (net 14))
 (segment (start 155.764999 109.805194) (end 156.460767 109.109426) (width 0.25) (layer F.Cu) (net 14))
 (segment (start 155.764999 110.457001) (end 155.764999 109.805194) (width 0.25) (layer F.Cu) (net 14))
 (segment (start 155.915 110.607002) (end 155.764999 110.457001) (width 0.25) (layer F.Cu) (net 14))
 (via (at 156.460767 109.109426) (size 0.8) (drill 0.4) (layers F.Cu B.Cu) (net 14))
 (segment (start 155.915 111.45) (end 155.915 110.607002) (width 0.25) (layer F.Cu) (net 14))
 (segment (start 155.764999 117.285001) (end 155.665001 117.384999) (width 0.25) (layer B.Cu) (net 14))
 (segment (start 155.764999 109.805194) (end 155.764999 117.285001) (width 0.25) (layer B.Cu) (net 14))
 (segment (start 156.460767 109.109426) (end 155.764999 109.805194) (width 0.25) (layer B.Cu) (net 14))
 (segment (start 155.265 111.45) (end 155.265 109.545) (width 0.25) (layer F.Cu) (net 13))
 (segment (start 155.265 109.545) (end 154.94 109.22) (width 0.25) (layer F.Cu) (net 13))
 (segment (start 154.94 109.22) (end 154.94 109.22) (width 0.25) (layer F.Cu) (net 13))
 (via (at 154.94 109.22) (size 0.8) (drill 0.4) (layers F.Cu B.Cu) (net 13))
 (segment (start 154.94 115.57) (end 148.59 121.92) (width 0.25) (layer B.Cu) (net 13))
 (segment (start 154.94 109.22) (end 154.94 115.57) (width 0.25) (layer B.Cu) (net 13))
 (segment (start 153.67 114.3) (end 146.05 121.92) (width 0.25) (layer B.Cu) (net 12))
 (via (at 154.215 110.236) (size 0.8) (drill 0.4) (layers F.Cu B.Cu) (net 12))
 (segment (start 154.615 110.636) (end 154.215 110.236) (width 0.25) (layer F.Cu) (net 12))
 (segment (start 154.615 111.45) (end 154.615 110.636) (width 0.25) (layer F.Cu) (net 12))
 (segment (start 153.67 110.781) (end 153.67 111.379) (width 0.25) (layer B.Cu) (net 12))
 (segment (start 154.215 110.236) (end 153.67 110.781) (width 0.25) (layer B.Cu) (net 12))
 (segment (start 153.67 111.379) (end 153.67 114.3) (width 0.25) (layer B.Cu) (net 12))
 (segment (start 148.190001 115.960003) (end 150.254999 118.025001) (width 0.25) (layer F.Cu) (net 28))
 (segment (start 148.209 110.109) (end 148.190001 110.127999) (width 0.25) (layer B.Cu) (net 28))
 (segment (start 151.365 117.835002) (end 151.365 117.15) (width 0.25) (layer F.Cu) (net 28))
 (segment (start 148.190001 110.127999) (end 148.190001 113.265001) (width 0.25) (layer B.Cu) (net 28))
 (segment (start 148.190001 113.265001) (end 148.190001 115.960003) (width 0.25) (layer F.Cu) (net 28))
 (segment (start 151.175001 118.025001) (end 151.365 117.835002) (width 0.25) (layer F.Cu) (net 28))
 (segment (start 150.254999 118.025001) (end 151.175001 118.025001) (width 0.25) (layer F.Cu) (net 28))
 (via (at 148.209 110.109) (size 0.8) (drill 0.4) (layers F.Cu B.Cu) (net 28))
 (via (at 148.190001 113.265001) (size 0.8) (drill 0.4) (layers F.Cu B.Cu) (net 28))
 (segment (start 148.209 108.331) (end 148.59 107.95) (width 0.25) (layer F.Cu) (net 28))
 (segment (start 148.209 110.109) (end 148.209 108.331) (width 0.25) (layer F.Cu) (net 28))
 (segment (start 151.365 110.65) (end 150.824 110.109) (width 0.25) (layer F.Cu) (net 10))
 (segment (start 151.365 111.45) (end 151.365 110.65) (width 0.25) (layer F.Cu) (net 10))
 (via (at 150.824 110.109) (size 0.8) (drill 0.4) (layers F.Cu B.Cu) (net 10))
 (segment (start 150.824 110.109) (end 149.225 111.708) (width 0.25) (layer B.Cu) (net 10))
 (via (at 149.225 111.708) (size 0.8) (drill 0.4) (layers F.Cu B.Cu) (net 10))
 (segment (start 147.7795 111.708) (end 147.7275 111.76) (width 0.25) (layer F.Cu) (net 10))
 (segment (start 149.225 111.708) (end 147.7795 111.708) (width 0.25) (layer F.Cu) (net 10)))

